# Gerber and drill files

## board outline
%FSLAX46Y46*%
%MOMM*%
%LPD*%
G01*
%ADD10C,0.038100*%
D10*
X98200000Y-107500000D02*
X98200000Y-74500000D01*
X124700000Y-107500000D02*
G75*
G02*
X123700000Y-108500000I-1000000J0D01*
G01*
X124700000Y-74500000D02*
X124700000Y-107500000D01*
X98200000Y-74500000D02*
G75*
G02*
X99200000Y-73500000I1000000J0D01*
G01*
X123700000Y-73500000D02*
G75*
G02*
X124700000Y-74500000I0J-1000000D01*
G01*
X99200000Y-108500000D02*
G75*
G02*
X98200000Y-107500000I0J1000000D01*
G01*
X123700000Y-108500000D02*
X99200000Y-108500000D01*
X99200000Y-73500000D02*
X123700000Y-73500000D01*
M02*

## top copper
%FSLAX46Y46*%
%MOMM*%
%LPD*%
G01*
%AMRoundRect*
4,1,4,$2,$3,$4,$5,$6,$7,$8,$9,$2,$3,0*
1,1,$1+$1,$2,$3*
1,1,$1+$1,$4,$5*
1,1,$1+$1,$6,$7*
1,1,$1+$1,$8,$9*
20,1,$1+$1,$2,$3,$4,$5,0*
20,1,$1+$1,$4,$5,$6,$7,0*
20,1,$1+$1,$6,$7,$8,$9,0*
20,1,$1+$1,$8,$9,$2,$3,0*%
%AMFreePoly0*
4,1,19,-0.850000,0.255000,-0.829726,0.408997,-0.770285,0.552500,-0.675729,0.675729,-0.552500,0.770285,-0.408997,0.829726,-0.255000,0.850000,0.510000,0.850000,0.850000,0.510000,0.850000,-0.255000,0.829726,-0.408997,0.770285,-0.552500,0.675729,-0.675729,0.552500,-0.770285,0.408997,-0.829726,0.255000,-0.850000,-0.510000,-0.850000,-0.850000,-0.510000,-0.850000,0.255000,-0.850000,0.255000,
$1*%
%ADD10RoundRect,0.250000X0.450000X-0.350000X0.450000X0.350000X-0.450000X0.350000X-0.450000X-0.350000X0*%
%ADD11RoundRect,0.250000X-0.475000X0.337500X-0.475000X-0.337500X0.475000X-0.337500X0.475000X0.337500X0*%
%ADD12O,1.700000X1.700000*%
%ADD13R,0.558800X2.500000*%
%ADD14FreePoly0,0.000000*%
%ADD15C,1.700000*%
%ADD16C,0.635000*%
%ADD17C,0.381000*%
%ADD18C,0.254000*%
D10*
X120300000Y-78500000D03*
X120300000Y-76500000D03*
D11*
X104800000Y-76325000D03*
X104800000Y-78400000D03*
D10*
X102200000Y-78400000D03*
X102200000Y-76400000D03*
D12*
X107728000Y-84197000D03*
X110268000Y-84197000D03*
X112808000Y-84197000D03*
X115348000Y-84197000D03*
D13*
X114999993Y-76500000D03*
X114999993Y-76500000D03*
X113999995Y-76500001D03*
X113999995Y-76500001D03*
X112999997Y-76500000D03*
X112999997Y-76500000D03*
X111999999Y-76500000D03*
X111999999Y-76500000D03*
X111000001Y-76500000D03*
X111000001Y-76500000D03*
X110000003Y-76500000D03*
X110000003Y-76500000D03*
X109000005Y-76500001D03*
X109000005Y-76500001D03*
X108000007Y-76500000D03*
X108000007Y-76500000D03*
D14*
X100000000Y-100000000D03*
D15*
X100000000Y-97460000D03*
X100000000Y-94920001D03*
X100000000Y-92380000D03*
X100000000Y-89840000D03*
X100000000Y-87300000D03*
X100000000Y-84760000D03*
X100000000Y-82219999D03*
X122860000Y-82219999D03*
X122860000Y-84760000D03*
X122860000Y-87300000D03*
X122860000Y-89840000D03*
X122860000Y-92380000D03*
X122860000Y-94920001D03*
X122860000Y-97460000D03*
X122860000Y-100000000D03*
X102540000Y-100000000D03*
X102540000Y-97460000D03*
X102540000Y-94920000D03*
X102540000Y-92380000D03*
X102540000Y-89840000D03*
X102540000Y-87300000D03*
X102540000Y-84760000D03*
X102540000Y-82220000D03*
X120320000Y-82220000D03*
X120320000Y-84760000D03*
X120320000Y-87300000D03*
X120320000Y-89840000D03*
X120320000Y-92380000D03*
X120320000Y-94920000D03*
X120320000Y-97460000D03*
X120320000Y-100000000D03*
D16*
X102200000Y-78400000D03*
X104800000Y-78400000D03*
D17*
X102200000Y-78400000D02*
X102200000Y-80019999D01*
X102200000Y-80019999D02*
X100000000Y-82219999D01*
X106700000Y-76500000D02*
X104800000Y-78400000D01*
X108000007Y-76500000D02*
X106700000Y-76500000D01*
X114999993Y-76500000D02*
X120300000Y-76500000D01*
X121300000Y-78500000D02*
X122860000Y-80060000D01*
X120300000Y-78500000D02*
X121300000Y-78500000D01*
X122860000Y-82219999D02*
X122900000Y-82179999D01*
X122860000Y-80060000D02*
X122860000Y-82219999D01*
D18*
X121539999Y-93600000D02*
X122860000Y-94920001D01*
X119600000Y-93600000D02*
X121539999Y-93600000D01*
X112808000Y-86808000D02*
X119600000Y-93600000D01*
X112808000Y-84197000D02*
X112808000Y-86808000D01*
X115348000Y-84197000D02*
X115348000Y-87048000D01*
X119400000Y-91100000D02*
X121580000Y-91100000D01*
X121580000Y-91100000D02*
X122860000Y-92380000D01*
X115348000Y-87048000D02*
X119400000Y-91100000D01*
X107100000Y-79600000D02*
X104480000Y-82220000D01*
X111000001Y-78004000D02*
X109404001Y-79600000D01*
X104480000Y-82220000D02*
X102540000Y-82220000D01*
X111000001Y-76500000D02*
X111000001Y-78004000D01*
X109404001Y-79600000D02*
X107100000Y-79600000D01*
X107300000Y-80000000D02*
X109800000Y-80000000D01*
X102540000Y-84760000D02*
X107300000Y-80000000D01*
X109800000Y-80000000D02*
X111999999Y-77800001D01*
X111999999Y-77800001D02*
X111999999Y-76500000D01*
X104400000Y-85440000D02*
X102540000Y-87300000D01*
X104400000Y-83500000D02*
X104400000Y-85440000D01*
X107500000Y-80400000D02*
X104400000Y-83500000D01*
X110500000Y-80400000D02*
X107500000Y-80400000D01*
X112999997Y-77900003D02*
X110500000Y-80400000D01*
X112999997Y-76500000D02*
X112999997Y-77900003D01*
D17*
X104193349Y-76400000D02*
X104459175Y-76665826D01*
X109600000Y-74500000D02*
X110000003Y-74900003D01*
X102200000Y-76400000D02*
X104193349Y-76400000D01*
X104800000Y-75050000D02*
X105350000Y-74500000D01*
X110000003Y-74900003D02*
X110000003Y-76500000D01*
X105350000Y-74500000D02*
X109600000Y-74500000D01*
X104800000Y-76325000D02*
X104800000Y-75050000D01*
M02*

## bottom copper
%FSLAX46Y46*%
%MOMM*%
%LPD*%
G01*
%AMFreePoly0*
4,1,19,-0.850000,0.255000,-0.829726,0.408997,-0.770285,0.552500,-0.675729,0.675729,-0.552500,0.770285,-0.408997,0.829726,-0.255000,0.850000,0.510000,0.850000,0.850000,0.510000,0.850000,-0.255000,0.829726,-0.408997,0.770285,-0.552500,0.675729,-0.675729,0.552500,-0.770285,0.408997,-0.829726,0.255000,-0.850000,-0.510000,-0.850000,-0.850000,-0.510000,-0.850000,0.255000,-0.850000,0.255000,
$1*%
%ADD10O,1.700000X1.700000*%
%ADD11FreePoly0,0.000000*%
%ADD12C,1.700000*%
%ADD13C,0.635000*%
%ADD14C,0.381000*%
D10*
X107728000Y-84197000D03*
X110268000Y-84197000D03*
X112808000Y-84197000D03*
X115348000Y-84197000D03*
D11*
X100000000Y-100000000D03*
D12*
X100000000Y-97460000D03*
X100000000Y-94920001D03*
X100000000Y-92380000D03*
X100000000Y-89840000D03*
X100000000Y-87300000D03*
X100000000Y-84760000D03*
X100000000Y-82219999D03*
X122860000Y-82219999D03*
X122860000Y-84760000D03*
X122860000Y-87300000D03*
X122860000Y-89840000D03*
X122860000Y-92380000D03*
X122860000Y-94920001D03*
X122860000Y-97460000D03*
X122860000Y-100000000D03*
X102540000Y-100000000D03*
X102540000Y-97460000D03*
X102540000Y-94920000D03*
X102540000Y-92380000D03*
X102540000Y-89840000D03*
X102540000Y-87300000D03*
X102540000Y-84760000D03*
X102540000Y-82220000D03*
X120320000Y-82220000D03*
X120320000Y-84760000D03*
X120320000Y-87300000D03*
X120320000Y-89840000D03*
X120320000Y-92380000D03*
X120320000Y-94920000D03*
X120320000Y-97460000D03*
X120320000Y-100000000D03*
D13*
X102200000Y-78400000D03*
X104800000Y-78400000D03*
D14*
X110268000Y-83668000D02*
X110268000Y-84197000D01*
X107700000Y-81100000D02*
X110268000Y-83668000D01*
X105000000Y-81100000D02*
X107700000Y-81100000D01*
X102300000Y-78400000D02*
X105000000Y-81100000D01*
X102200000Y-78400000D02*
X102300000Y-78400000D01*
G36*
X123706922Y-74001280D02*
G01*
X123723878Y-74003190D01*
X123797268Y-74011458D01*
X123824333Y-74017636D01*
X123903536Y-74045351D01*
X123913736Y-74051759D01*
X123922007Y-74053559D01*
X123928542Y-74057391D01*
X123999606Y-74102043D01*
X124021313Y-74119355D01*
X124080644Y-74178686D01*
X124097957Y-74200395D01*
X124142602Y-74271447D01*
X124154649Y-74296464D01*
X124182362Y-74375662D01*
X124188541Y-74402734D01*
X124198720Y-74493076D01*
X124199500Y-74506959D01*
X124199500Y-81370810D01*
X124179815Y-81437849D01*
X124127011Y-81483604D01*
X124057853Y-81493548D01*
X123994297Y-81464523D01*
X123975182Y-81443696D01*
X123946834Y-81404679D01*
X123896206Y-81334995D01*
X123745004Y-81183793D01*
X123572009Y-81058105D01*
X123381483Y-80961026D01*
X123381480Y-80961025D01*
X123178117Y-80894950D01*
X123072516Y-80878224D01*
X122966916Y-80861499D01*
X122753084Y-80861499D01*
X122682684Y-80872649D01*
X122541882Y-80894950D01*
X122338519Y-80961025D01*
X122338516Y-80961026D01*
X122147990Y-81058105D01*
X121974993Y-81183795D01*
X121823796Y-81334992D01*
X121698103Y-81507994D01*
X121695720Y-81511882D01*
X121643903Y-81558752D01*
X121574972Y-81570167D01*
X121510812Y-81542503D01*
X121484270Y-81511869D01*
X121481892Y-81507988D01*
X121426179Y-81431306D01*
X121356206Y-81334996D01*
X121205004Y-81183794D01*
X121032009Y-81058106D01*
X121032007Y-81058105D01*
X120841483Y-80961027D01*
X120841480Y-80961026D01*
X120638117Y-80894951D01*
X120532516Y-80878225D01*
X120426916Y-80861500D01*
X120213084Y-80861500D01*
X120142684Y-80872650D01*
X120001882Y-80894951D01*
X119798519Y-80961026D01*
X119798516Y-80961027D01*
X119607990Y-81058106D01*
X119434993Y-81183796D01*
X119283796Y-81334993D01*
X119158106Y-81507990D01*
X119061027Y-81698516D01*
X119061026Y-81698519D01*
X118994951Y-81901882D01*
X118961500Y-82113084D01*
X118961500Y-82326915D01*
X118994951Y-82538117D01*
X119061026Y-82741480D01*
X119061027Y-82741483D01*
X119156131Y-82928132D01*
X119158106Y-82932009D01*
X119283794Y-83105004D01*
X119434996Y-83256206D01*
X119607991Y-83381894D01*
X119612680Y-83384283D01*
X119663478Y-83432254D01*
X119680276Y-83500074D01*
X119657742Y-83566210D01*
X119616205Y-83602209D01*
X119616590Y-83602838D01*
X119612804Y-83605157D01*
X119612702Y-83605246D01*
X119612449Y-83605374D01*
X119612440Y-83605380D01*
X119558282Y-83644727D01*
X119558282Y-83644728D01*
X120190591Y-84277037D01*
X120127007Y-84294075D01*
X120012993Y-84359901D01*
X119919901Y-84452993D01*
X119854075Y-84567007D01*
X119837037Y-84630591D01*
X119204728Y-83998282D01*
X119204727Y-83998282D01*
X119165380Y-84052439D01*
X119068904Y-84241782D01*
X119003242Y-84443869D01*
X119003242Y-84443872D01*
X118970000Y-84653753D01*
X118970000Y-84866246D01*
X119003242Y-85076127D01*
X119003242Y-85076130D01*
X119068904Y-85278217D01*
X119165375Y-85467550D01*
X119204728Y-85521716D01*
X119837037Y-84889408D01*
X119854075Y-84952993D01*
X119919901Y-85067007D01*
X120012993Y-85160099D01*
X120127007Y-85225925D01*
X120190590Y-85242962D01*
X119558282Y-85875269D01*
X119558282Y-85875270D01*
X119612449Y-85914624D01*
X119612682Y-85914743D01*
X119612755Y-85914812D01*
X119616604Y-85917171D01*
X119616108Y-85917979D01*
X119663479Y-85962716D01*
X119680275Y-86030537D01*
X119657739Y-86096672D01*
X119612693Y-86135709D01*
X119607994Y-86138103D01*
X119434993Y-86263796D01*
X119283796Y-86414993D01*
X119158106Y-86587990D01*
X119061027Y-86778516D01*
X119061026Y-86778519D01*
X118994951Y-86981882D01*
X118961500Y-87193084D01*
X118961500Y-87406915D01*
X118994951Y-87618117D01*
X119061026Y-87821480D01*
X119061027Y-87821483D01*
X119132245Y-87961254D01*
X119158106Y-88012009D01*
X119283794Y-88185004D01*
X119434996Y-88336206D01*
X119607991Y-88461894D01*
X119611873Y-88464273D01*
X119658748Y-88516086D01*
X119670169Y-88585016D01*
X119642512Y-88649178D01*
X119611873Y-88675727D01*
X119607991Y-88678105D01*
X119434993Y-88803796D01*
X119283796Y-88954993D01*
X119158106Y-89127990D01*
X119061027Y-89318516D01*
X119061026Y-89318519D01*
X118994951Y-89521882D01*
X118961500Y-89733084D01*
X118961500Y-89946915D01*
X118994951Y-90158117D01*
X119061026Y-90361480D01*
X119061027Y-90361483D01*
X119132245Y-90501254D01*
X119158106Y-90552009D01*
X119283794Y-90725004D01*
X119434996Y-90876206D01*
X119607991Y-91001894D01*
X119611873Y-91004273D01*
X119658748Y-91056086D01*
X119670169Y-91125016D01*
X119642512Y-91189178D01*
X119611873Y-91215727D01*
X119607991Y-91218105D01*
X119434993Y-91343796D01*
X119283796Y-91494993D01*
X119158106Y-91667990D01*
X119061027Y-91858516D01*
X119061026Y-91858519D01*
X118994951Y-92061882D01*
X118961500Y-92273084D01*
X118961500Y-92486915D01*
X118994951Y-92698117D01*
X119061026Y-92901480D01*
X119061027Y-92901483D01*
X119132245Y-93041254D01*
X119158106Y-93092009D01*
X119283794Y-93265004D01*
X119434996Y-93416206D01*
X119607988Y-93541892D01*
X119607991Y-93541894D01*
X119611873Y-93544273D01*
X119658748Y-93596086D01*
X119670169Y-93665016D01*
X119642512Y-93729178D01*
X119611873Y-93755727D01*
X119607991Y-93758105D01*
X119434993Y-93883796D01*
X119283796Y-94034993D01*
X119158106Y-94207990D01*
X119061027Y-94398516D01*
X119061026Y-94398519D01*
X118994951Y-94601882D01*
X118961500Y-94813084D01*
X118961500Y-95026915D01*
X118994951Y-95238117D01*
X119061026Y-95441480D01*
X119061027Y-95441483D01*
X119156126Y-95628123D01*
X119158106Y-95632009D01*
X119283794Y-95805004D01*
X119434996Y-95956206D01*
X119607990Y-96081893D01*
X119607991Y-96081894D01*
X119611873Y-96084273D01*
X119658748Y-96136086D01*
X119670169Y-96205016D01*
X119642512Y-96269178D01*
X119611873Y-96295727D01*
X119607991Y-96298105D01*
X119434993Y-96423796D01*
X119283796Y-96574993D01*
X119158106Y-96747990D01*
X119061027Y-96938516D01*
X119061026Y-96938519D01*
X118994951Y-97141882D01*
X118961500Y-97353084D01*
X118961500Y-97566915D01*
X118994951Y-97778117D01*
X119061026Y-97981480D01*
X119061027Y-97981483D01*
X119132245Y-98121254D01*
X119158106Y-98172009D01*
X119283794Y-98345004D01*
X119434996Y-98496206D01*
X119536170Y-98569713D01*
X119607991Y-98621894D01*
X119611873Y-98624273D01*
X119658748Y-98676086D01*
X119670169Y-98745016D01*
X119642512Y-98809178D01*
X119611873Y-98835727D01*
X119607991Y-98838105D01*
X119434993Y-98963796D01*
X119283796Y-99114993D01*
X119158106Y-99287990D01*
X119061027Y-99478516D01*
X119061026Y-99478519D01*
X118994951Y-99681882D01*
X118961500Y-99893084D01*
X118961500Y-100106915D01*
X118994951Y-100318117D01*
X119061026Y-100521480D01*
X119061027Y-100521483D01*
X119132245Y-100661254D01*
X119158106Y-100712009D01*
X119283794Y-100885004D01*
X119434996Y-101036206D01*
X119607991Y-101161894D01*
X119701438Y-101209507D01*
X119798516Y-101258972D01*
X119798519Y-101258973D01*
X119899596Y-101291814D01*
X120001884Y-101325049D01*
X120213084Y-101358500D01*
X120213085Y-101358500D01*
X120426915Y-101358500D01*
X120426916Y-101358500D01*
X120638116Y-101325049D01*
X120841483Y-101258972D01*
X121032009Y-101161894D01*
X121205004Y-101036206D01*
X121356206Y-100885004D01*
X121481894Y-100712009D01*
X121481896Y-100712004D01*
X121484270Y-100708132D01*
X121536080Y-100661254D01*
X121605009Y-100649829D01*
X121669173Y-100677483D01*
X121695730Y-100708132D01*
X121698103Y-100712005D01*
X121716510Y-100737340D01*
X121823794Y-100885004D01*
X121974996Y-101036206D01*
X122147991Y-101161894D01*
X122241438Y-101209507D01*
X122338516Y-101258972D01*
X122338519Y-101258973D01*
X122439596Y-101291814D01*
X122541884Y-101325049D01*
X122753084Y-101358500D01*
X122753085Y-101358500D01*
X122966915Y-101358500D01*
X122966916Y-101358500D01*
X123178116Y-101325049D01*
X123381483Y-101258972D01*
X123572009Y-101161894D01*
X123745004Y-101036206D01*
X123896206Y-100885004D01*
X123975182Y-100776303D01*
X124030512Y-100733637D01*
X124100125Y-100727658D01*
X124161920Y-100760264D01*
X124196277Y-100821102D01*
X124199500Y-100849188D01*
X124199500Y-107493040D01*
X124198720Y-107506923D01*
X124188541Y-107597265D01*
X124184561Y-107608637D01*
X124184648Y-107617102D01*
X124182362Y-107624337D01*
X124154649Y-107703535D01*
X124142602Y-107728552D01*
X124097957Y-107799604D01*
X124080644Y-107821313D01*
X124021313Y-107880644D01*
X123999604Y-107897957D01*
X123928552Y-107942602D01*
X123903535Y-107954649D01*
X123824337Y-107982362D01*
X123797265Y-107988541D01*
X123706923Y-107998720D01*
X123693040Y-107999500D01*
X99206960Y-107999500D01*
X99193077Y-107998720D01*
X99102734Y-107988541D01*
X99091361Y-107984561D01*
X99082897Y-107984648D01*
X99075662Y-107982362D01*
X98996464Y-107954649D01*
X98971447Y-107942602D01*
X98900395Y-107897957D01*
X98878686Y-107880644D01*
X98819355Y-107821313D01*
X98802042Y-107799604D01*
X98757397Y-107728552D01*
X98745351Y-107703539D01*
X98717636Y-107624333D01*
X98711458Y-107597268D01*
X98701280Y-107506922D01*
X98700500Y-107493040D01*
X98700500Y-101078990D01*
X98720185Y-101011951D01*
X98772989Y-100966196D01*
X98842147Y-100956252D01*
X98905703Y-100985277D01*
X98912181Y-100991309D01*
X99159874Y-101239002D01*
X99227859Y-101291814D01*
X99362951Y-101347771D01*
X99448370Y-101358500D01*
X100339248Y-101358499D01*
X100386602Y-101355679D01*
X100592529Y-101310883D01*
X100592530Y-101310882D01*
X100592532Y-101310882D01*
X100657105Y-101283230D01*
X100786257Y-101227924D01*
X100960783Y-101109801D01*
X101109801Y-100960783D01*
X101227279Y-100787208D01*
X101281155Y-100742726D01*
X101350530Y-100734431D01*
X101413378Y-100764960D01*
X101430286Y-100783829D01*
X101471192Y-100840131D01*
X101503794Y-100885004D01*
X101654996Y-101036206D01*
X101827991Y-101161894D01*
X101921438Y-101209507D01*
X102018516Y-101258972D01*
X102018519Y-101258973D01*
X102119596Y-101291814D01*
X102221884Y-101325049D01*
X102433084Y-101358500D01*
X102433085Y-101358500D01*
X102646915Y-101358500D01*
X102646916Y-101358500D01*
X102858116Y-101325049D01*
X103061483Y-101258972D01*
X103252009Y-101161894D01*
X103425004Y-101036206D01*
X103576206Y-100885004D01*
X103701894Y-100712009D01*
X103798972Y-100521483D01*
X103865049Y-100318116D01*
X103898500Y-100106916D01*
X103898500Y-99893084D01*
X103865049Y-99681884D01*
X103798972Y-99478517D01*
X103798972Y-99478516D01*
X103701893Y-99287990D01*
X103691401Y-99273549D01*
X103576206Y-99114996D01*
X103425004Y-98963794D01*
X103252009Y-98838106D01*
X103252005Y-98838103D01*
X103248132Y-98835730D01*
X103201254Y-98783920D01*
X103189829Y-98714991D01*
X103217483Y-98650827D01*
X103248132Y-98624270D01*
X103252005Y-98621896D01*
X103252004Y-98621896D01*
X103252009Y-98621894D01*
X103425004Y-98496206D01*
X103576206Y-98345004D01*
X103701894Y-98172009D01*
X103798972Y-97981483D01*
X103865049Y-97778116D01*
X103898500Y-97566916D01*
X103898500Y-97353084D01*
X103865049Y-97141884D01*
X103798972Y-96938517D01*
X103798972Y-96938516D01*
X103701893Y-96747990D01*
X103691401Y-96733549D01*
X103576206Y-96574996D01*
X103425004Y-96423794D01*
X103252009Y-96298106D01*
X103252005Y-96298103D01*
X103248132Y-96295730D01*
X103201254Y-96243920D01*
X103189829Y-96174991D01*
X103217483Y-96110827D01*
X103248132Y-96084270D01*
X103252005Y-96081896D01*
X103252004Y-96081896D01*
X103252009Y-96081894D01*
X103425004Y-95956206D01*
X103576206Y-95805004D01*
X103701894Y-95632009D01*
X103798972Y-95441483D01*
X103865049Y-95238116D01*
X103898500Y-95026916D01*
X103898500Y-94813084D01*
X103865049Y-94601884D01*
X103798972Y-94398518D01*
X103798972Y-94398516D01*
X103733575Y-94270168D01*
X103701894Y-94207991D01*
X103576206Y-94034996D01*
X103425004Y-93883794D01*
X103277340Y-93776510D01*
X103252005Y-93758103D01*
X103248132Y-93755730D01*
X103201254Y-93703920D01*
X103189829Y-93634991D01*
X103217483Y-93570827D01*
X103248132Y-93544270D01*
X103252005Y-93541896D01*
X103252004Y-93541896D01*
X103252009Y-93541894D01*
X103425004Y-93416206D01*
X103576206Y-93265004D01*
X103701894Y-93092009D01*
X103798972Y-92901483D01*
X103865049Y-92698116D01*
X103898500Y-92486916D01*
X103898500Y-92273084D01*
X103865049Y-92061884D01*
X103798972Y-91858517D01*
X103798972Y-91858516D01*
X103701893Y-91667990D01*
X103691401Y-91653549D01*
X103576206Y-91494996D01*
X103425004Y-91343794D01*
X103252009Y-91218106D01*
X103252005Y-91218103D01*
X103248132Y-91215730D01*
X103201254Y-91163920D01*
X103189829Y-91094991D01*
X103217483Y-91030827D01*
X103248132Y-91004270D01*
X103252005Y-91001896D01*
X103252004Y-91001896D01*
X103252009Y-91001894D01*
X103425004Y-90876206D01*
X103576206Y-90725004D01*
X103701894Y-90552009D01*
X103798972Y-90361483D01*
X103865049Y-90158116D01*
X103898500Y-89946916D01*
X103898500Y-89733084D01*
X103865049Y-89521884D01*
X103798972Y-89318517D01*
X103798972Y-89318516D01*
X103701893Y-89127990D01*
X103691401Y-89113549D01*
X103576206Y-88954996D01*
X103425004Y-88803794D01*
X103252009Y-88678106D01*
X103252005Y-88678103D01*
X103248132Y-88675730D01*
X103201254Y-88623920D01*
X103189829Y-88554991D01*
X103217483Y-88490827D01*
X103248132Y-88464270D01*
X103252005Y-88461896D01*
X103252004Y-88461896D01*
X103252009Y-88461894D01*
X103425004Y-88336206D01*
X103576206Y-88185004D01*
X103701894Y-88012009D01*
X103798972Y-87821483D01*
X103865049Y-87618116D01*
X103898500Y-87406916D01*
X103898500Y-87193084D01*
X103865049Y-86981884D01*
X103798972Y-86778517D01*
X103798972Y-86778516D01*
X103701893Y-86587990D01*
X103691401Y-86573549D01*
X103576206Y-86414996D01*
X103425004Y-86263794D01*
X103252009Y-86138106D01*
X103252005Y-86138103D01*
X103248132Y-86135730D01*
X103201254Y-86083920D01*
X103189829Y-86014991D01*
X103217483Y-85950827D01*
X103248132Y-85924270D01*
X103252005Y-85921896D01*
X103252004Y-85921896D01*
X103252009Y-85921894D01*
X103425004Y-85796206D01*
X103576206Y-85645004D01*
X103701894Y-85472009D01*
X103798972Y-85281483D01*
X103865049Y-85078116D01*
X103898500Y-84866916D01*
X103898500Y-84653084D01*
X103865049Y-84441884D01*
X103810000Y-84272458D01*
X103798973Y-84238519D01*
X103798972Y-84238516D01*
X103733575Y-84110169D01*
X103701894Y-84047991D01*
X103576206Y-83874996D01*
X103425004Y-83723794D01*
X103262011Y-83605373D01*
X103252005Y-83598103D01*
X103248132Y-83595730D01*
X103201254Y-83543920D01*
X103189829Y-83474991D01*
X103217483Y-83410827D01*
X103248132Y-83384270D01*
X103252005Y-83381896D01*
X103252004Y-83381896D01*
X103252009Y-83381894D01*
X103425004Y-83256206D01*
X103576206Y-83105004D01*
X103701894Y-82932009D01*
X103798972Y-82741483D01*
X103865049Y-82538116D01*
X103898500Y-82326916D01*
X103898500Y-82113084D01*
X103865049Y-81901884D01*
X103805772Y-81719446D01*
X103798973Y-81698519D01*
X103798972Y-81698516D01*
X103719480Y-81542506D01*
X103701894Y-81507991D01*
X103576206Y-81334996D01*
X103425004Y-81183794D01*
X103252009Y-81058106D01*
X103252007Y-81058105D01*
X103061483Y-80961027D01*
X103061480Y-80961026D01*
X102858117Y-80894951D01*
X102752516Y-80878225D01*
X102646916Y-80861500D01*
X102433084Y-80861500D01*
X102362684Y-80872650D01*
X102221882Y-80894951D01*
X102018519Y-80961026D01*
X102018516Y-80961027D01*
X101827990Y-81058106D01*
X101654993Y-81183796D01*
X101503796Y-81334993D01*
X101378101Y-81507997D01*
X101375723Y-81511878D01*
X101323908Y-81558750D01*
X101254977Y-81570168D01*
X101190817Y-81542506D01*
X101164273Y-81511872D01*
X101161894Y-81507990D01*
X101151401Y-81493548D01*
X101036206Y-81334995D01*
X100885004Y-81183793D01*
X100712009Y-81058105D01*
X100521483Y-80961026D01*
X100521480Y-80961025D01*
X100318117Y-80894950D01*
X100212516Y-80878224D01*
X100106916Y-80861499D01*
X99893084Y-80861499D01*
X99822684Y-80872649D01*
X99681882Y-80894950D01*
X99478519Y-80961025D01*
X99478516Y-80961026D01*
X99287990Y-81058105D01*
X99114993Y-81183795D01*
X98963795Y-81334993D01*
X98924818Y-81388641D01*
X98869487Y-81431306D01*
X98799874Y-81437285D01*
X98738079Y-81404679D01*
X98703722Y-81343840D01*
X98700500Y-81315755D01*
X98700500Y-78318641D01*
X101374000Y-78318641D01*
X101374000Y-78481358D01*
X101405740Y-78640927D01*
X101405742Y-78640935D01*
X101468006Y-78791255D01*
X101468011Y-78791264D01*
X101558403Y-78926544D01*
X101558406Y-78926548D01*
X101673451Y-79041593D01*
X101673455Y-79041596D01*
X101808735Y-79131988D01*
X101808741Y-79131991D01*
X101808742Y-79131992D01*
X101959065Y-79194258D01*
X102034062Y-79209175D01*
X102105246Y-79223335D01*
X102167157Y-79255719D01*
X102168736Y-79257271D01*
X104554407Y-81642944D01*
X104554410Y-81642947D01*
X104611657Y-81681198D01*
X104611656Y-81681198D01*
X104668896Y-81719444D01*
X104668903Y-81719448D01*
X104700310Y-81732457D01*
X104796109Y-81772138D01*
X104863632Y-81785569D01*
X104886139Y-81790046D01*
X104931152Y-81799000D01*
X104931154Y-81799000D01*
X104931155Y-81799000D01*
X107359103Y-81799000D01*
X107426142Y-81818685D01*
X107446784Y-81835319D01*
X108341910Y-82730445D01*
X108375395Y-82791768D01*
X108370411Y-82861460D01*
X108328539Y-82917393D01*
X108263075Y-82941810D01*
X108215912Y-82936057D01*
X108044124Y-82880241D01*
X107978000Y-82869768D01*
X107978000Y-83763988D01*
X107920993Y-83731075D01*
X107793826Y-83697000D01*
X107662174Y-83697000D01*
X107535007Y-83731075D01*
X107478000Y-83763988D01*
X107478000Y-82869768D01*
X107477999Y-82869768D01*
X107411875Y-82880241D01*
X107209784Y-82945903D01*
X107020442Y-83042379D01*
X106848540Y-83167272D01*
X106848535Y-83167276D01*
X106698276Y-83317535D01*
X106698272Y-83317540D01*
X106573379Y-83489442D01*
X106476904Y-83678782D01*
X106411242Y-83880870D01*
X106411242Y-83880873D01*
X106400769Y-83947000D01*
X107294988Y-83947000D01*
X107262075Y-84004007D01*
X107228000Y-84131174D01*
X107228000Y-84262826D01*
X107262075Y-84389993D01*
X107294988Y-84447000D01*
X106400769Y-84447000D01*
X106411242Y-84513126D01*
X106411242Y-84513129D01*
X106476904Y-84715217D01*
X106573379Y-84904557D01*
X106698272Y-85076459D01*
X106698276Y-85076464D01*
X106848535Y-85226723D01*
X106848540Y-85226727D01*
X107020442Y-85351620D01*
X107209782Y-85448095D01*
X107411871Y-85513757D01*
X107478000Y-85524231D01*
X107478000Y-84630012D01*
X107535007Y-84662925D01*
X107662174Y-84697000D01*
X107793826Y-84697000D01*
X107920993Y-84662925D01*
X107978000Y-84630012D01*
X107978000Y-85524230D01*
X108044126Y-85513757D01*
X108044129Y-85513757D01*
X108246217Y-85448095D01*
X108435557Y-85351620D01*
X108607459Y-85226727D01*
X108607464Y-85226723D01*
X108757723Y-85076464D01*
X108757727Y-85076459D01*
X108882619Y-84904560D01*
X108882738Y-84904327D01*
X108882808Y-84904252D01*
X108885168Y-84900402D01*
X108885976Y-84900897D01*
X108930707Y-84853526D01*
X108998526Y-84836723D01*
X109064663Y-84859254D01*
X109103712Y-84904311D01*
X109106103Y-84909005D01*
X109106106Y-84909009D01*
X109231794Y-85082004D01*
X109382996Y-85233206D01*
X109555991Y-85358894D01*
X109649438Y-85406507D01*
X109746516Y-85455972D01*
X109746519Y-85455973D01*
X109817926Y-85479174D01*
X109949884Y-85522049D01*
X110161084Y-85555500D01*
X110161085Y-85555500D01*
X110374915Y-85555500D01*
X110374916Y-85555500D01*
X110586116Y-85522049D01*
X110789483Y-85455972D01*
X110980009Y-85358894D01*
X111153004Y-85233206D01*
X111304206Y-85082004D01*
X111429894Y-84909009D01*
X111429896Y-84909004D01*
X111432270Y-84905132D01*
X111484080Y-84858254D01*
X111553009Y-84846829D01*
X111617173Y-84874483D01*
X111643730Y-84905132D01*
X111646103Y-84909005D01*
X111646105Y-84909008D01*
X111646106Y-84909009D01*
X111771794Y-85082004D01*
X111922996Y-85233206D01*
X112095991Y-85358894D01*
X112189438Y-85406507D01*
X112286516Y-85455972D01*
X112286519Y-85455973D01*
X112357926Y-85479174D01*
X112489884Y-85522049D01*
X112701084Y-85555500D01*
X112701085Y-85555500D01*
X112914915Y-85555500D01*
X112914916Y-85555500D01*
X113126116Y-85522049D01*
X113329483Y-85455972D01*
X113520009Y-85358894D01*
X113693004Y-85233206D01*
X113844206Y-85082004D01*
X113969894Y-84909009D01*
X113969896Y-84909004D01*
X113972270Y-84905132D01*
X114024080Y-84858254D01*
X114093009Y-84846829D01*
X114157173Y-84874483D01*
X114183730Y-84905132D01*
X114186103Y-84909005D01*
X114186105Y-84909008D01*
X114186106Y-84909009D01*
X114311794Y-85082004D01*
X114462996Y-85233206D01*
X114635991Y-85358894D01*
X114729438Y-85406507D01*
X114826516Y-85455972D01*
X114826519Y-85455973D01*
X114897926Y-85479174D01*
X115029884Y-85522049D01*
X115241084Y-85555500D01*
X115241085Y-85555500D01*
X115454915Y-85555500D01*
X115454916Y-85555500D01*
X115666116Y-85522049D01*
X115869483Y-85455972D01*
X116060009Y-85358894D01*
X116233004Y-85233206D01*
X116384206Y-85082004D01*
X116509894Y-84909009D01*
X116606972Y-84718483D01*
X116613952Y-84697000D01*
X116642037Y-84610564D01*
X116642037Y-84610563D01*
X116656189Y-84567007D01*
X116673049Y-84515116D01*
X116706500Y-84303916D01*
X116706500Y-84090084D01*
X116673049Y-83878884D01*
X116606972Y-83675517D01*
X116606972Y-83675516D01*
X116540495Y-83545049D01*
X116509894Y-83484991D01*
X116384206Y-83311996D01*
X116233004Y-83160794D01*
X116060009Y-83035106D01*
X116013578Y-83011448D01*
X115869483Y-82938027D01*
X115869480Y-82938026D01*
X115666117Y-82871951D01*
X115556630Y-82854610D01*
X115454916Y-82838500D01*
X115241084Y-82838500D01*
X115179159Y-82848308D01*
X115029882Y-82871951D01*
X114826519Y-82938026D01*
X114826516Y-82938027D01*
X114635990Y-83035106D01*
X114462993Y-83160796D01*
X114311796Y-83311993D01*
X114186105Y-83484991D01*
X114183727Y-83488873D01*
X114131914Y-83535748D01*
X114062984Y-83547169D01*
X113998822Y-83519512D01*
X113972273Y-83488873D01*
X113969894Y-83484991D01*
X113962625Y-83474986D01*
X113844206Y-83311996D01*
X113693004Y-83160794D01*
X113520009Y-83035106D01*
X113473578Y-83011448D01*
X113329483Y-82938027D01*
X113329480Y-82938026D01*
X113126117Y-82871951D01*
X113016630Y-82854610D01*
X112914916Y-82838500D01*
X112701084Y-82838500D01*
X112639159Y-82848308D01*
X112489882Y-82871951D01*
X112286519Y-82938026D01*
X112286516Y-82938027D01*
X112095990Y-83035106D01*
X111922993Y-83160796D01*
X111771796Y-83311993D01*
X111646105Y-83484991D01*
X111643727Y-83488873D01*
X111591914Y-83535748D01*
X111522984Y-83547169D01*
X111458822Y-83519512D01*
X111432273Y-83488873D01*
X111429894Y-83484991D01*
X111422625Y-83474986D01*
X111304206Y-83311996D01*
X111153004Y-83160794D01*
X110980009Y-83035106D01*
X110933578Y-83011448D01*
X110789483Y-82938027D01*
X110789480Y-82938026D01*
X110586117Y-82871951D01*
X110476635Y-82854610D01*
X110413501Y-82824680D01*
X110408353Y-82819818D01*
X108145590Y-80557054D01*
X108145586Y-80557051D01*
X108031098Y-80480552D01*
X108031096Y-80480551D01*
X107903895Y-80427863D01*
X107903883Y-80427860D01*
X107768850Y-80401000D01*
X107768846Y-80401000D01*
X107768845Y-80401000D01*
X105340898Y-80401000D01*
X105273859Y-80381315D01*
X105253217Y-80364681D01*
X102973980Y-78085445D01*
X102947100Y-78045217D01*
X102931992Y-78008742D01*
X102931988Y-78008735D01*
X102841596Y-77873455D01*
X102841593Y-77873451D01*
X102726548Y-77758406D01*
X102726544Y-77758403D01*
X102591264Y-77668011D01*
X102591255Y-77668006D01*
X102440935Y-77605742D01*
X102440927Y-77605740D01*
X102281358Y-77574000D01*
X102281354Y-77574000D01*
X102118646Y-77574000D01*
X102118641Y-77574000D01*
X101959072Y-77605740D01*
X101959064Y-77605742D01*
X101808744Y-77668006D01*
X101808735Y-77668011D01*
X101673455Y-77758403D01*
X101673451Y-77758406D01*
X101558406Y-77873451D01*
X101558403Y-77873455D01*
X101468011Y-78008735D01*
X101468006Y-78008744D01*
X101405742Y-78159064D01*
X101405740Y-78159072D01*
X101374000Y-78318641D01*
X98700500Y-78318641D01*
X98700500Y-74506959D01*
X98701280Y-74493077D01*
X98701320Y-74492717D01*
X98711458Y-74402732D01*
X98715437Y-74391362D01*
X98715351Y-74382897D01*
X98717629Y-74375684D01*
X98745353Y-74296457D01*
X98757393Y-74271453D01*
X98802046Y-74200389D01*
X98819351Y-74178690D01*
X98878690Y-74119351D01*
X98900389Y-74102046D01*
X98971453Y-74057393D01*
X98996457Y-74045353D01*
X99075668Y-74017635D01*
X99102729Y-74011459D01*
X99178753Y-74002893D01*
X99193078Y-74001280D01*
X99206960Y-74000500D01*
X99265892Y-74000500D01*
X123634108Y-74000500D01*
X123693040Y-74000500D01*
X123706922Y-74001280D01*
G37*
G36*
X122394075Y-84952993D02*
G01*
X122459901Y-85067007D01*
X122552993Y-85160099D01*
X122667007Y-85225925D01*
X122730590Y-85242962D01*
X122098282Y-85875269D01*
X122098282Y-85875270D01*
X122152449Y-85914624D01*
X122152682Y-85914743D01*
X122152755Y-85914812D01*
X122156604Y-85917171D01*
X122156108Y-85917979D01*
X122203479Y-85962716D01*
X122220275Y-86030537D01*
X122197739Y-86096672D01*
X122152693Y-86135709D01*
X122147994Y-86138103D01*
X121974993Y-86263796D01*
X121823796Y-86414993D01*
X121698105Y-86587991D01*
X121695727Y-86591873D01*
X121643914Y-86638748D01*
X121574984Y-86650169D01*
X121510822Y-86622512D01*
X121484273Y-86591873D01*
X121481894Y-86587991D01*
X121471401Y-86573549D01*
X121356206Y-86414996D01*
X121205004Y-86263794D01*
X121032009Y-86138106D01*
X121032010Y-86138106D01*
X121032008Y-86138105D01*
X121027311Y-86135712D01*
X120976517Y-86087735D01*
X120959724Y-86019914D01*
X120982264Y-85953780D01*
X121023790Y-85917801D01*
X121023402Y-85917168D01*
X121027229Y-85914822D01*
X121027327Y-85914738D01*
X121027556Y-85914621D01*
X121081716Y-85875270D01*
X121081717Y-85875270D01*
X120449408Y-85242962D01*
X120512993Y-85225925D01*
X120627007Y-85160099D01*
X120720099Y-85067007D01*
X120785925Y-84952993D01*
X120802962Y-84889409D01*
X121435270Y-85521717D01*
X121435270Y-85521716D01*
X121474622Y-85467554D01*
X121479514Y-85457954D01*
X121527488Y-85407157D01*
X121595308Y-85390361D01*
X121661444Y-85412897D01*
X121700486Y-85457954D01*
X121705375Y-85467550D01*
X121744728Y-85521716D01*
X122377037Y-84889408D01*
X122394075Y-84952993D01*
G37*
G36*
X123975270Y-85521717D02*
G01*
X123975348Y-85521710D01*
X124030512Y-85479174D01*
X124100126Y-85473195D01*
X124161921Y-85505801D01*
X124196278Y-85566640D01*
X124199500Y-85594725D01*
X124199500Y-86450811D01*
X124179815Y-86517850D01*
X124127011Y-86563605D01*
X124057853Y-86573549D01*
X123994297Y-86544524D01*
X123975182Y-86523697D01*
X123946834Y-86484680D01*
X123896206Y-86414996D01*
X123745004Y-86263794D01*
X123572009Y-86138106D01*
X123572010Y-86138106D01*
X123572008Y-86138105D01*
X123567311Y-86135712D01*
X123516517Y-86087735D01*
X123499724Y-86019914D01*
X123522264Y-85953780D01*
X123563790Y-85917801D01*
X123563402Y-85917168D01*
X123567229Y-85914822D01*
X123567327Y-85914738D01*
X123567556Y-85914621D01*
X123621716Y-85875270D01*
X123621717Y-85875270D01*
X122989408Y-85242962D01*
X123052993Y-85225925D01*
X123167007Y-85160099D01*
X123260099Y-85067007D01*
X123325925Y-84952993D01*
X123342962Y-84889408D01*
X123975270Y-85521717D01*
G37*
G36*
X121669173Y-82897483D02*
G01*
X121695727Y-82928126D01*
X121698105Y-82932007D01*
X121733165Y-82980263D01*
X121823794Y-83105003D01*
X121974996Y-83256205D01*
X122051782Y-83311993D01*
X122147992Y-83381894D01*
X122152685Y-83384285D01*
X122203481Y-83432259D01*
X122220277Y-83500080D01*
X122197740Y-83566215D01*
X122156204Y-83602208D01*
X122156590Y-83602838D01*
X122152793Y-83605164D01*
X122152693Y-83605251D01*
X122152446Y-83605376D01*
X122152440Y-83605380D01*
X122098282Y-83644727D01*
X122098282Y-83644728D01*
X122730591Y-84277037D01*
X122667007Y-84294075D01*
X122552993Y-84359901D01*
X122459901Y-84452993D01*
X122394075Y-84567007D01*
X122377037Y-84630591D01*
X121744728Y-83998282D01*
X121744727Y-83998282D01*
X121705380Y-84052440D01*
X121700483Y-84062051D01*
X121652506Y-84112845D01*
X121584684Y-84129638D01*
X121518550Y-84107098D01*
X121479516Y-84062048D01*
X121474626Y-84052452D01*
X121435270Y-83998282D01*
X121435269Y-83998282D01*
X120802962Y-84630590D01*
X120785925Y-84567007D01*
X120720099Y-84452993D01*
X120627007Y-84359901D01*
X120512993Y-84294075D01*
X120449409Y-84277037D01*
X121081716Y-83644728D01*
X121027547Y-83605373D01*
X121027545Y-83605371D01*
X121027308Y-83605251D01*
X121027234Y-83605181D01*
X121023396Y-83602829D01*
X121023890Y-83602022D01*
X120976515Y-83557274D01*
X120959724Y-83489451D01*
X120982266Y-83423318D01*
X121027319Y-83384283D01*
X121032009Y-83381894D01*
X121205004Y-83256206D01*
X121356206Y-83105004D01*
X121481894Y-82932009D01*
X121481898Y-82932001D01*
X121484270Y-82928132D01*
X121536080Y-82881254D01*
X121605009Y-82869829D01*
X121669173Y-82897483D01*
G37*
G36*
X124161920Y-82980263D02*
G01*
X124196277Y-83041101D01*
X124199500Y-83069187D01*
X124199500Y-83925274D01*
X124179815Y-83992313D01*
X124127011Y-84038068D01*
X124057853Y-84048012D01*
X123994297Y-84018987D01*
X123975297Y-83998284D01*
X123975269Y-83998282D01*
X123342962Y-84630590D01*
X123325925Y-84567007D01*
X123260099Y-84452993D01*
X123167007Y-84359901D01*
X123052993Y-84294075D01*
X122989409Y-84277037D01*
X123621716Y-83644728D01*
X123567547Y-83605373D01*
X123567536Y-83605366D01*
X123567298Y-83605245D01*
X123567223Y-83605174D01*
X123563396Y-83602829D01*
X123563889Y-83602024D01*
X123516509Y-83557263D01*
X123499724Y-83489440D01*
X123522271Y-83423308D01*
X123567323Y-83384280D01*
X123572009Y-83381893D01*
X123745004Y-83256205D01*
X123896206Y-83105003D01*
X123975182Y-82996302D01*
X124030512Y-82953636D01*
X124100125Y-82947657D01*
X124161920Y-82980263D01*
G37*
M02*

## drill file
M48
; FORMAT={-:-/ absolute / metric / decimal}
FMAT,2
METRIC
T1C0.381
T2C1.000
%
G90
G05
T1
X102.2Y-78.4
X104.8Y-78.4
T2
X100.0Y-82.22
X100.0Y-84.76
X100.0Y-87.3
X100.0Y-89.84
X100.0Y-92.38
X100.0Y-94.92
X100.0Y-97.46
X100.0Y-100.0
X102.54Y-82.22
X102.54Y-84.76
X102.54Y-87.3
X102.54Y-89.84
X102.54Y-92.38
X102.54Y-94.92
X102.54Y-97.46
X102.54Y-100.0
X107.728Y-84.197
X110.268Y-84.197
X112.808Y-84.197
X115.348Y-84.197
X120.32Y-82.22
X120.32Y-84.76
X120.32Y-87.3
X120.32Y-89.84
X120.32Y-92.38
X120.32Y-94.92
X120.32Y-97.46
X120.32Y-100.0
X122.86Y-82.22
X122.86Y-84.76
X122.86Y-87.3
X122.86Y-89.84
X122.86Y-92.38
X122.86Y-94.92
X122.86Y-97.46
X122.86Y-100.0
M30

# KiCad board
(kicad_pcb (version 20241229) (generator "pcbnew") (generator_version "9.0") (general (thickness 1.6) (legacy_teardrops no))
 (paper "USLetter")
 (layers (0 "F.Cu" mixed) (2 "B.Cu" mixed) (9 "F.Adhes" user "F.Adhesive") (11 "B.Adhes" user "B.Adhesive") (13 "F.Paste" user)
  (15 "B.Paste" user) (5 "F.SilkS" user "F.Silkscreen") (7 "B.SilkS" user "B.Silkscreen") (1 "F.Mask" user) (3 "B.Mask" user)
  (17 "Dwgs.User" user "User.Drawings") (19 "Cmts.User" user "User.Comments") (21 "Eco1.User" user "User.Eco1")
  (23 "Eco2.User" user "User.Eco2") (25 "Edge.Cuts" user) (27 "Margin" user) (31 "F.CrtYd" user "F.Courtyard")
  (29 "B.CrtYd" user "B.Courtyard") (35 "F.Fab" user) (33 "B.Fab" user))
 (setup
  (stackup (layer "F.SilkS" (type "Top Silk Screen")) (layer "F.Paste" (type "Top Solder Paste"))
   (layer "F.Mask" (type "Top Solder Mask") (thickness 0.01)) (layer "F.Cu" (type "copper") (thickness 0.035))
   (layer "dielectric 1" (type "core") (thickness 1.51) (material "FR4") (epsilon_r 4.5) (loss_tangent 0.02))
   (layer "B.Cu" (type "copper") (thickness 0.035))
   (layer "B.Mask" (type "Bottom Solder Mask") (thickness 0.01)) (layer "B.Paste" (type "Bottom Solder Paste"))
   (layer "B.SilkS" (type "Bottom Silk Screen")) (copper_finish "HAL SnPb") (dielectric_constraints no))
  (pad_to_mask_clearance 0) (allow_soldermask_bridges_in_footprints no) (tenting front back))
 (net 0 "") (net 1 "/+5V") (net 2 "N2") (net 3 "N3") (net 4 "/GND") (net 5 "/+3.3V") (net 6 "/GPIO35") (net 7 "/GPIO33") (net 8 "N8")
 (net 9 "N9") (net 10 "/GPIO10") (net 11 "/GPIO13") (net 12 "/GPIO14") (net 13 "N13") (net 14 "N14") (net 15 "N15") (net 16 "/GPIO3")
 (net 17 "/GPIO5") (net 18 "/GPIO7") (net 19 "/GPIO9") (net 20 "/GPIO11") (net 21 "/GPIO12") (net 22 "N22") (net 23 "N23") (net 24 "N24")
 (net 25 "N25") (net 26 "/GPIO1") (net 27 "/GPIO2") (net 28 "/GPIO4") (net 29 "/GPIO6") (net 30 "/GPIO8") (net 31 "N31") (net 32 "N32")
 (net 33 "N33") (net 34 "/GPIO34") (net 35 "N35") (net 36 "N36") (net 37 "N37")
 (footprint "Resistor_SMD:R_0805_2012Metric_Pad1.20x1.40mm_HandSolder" (layer "F.Cu") (at 120.3 77.5 90)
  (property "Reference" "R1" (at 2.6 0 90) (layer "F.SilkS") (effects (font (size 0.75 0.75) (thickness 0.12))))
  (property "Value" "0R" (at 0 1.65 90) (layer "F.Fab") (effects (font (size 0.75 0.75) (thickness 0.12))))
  (pad "1" smd roundrect (at -1 0 90) (size 1.2 1.4) (layers "F.Cu" "F.Mask" "F.Paste") (roundrect_rratio 0.208333) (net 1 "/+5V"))
  (pad "2" smd roundrect (at 1 0 90) (size 1.2 1.4) (layers "F.Cu" "F.Mask" "F.Paste") (roundrect_rratio 0.208333) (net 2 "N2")))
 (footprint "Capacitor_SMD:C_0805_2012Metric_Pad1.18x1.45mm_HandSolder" (layer "F.Cu") (at 104.8 77.3625 -90)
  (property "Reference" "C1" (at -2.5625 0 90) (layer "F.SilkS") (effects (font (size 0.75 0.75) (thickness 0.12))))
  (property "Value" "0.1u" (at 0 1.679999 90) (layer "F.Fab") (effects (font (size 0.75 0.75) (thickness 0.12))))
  (pad "1" smd roundrect (at -1.0375 0 270) (size 1.175 1.45) (layers "F.Cu" "F.Mask" "F.Paste") (roundrect_rratio 0.212766) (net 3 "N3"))
  (pad "2" smd roundrect (at 1.0375 0 270) (size 1.175 1.45) (layers "F.Cu" "F.Mask" "F.Paste") (roundrect_rratio 0.212766) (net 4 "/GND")))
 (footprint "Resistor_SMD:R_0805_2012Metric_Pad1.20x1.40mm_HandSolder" (layer "F.Cu") (at 102.2 77.4 90)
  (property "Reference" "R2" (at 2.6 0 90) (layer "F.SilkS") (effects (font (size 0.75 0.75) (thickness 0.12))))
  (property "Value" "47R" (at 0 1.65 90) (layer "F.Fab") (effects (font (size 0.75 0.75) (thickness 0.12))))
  (pad "1" smd roundrect (at -1 0 90) (size 1.2 1.4) (layers "F.Cu" "F.Mask" "F.Paste") (roundrect_rratio 0.208333) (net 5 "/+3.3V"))
  (pad "2" smd roundrect (at 1 0 90) (size 1.2 1.4) (layers "F.Cu" "F.Mask" "F.Paste") (roundrect_rratio 0.208333) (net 3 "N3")))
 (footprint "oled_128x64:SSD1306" (layer "F.Cu") (at 111.538 93.849)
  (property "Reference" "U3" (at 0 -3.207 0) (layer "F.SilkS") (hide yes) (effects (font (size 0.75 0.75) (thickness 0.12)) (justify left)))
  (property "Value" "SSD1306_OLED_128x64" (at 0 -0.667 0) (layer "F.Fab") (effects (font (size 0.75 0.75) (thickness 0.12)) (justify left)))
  (pad "1" thru_hole oval (at -3.81 -9.652 90) (size 1.7 1.7) (drill oval 1) (layers "*.Cu" "*.Mask") (remove_unused_layers no)
   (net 4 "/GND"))
  (pad "2" thru_hole oval (at -1.27 -9.652 90) (size 1.7 1.7) (drill oval 1) (layers "*.Cu" "*.Mask") (remove_unused_layers no)
   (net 5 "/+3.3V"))
  (pad "3" thru_hole oval (at 1.27 -9.652 90) (size 1.7 1.7) (drill oval 1) (layers "*.Cu" "*.Mask") (remove_unused_layers no)
   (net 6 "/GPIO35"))
  (pad "4" thru_hole oval (at 3.81 -9.652 90) (size 1.7 1.7) (drill oval 1) (layers "*.Cu" "*.Mask") (remove_unused_layers no)
   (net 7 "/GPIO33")))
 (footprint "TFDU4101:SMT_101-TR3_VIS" (layer "F.Cu") (at 111.5 75.6999 90)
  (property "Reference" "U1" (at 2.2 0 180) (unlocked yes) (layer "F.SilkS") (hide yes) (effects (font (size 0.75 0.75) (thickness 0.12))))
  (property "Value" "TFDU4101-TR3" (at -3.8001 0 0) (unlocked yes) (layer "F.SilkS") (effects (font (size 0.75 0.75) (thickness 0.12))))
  (pad "1" smd rect (at -0.8001 3.499993 90) (size 2.5 0.5588) (layers "F.Cu" "F.Mask" "F.Paste") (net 2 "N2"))
  (pad "1" smd rect (at -0.8001 3.499993 90) (size 2.5 0.5588) (layers "F.Cu" "F.Mask" "F.Paste") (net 2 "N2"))
  (pad "2" smd rect (at -0.800101 2.499995 90) (size 2.5 0.5588) (layers "F.Cu" "F.Mask" "F.Paste") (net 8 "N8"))
  (pad "2" smd rect (at -0.800101 2.499995 90) (size 2.5 0.5588) (layers "F.Cu" "F.Mask" "F.Paste") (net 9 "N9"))
  (pad "3" smd rect (at -0.8001 1.499997 90) (size 2.5 0.5588) (layers "F.Cu" "F.Mask" "F.Paste") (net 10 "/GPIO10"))
  (pad "3" smd rect (at -0.8001 1.499997 90) (size 2.5 0.5588) (layers "F.Cu" "F.Mask" "F.Paste") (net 10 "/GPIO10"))
  (pad "4" smd rect (at -0.8001 0.499999 90) (size 2.5 0.5588) (layers "F.Cu" "F.Mask" "F.Paste") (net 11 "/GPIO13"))
  (pad "4" smd rect (at -0.8001 0.499999 90) (size 2.5 0.5588) (layers "F.Cu" "F.Mask" "F.Paste") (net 11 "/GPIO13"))
  (pad "5" smd rect (at -0.8001 -0.499999 90) (size 2.5 0.5588) (layers "F.Cu" "F.Mask" "F.Paste") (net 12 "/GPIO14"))
  (pad "5" smd rect (at -0.8001 -0.499999 90) (size 2.5 0.5588) (layers "F.Cu" "F.Mask" "F.Paste") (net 12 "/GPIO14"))
  (pad "6" smd rect (at -0.8001 -1.499997 90) (size 2.5 0.5588) (layers "F.Cu" "F.Mask" "F.Paste") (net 3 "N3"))
  (pad "6" smd rect (at -0.8001 -1.499997 90) (size 2.5 0.5588) (layers "F.Cu" "F.Mask" "F.Paste") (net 3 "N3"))
  (pad "7" smd rect (at -0.800101 -2.499995 90) (size 2.5 0.5588) (layers "F.Cu" "F.Mask" "F.Paste") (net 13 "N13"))
  (pad "7" smd rect (at -0.800101 -2.499995 90) (size 2.5 0.5588) (layers "F.Cu" "F.Mask" "F.Paste") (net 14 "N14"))
  (pad "8" smd rect (at -0.8001 -3.499993 90) (size 2.5 0.5588) (layers "F.Cu" "F.Mask" "F.Paste") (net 4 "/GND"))
  (pad "8" smd rect (at -0.8001 -3.499993 90) (size 2.5 0.5588) (layers "F.Cu" "F.Mask" "F.Paste") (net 4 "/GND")))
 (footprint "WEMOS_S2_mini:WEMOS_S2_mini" (layer "B.Cu") (at 100 100)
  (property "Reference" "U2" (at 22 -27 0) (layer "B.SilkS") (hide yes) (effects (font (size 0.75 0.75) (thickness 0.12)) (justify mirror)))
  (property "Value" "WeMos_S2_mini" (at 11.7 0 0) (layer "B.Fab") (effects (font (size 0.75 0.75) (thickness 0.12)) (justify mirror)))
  (pad "1" thru_hole roundrect (at 0 0) (size 1.7 1.7) (drill 1) (layers "*.Cu" "*.Mask") (remove_unused_layers no) (roundrect_rratio 0.35)
   (chamfer_ratio 0.2) (chamfer top_right bottom_left) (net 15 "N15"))
  (pad "2" thru_hole circle (at 0 -2.54) (size 1.7 1.7) (drill 1) (layers "*.Cu" "*.Mask") (remove_unused_layers no) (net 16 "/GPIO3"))
  (pad "3" thru_hole circle (at 0 -5.079999) (size 1.7 1.7) (drill 1) (layers "*.Cu" "*.Mask") (remove_unused_layers no) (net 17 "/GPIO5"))
  (pad "4" thru_hole circle (at 0 -7.62) (size 1.7 1.7) (drill 1) (layers "*.Cu" "*.Mask") (remove_unused_layers no) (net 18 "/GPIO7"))
  (pad "5" thru_hole circle (at 0 -10.16) (size 1.7 1.7) (drill 1) (layers "*.Cu" "*.Mask") (remove_unused_layers no) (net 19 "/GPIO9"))
  (pad "6" thru_hole circle (at 0 -12.7) (size 1.7 1.7) (drill 1) (layers "*.Cu" "*.Mask") (remove_unused_layers no) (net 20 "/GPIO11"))
  (pad "7" thru_hole circle (at 0 -15.24) (size 1.7 1.7) (drill 1) (layers "*.Cu" "*.Mask") (remove_unused_layers no) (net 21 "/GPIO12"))
  (pad "8" thru_hole circle (at 0 -17.780001) (size 1.7 1.7) (drill 1) (layers "*.Cu" "*.Mask") (remove_unused_layers no) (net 5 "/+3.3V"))
  (pad "9" thru_hole circle (at 22.86 -17.780001) (size 1.7 1.7) (drill 1) (layers "*.Cu" "*.Mask") (remove_unused_layers no) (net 1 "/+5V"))
  (pad "10" thru_hole circle (at 22.86 -15.24) (size 1.7 1.7) (drill 1) (layers "*.Cu" "*.Mask") (remove_unused_layers no) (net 4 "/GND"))
  (pad "11" thru_hole circle (at 22.86 -12.7) (size 1.7 1.7) (drill 1) (layers "*.Cu" "*.Mask") (remove_unused_layers no) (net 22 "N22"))
  (pad "12" thru_hole circle (at 22.86 -10.16) (size 1.7 1.7) (drill 1) (layers "*.Cu" "*.Mask") (remove_unused_layers no) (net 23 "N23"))
  (pad "13" thru_hole circle (at 22.86 -7.62) (size 1.7 1.7) (drill 1) (layers "*.Cu" "*.Mask") (remove_unused_layers no) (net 7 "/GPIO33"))
  (pad "14" thru_hole circle (at 22.86 -5.079999) (size 1.7 1.7) (drill 1) (layers "*.Cu" "*.Mask") (remove_unused_layers no)
   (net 6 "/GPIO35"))
  (pad "15" thru_hole circle (at 22.86 -2.54) (size 1.7 1.7) (drill 1) (layers "*.Cu" "*.Mask") (remove_unused_layers no) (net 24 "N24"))
  (pad "16" thru_hole circle (at 22.86 0) (size 1.7 1.7) (drill 1) (layers "*.Cu" "*.Mask") (remove_unused_layers no) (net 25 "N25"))
  (pad "17" thru_hole circle (at 2.54 0) (size 1.7 1.7) (drill 1) (layers "*.Cu" "*.Mask") (remove_unused_layers no) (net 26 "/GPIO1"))
  (pad "18" thru_hole circle (at 2.54 -2.54) (size 1.7 1.7) (drill 1) (layers "*.Cu" "*.Mask") (remove_unused_layers no) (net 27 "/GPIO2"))
  (pad "19" thru_hole circle (at 2.54 -5.08) (size 1.7 1.7) (drill 1) (layers "*.Cu" "*.Mask") (remove_unused_layers no) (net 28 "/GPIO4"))
  (pad "20" thru_hole circle (at 2.54 -7.62) (size 1.7 1.7) (drill 1) (layers "*.Cu" "*.Mask") (remove_unused_layers no) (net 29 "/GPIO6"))
  (pad "21" thru_hole circle (at 2.54 -10.16) (size 1.7 1.7) (drill 1) (layers "*.Cu" "*.Mask") (remove_unused_layers no) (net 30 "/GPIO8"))
  (pad "22" thru_hole circle (at 2.54 -12.7) (size 1.7 1.7) (drill 1) (layers "*.Cu" "*.Mask") (remove_unused_layers no) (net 10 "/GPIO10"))
  (pad "23" thru_hole circle (at 2.54 -15.24) (size 1.7 1.7) (drill 1) (layers "*.Cu" "*.Mask") (remove_unused_layers no) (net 11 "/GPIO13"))
  (pad "24" thru_hole circle (at 2.54 -17.78) (size 1.7 1.7) (drill 1) (layers "*.Cu" "*.Mask") (remove_unused_layers no) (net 12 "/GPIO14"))
  (pad "25" thru_hole circle (at 20.32 -17.78) (size 1.7 1.7) (drill 1) (layers "*.Cu" "*.Mask") (remove_unused_layers no) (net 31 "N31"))
  (pad "26" thru_hole circle (at 20.32 -15.24) (size 1.7 1.7) (drill 1) (layers "*.Cu" "*.Mask") (remove_unused_layers no) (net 4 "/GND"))
  (pad "27" thru_hole circle (at 20.32 -12.7) (size 1.7 1.7) (drill 1) (layers "*.Cu" "*.Mask") (remove_unused_layers no) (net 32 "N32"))
  (pad "28" thru_hole circle (at 20.32 -10.16) (size 1.7 1.7) (drill 1) (layers "*.Cu" "*.Mask") (remove_unused_layers no) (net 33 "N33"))
  (pad "29" thru_hole circle (at 20.32 -7.62) (size 1.7 1.7) (drill 1) (layers "*.Cu" "*.Mask") (remove_unused_layers no) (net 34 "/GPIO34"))
  (pad "30" thru_hole circle (at 20.32 -5.08) (size 1.7 1.7) (drill 1) (layers "*.Cu" "*.Mask") (remove_unused_layers no) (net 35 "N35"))
  (pad "31" thru_hole circle (at 20.32 -2.54) (size 1.7 1.7) (drill 1) (layers "*.Cu" "*.Mask") (remove_unused_layers no) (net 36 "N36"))
  (pad "32" thru_hole circle (at 20.32 0) (size 1.7 1.7) (drill 1) (layers "*.Cu" "*.Mask") (remove_unused_layers no) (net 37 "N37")))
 (gr_line (start 98.2 107.5) (end 98.2 74.5) (stroke (width 0.0381) (type default)) (layer "Edge.Cuts"))
 (gr_arc (start 124.7 107.5) (mid 124.407107 108.207107) (end 123.7 108.5) (stroke (width 0.0381) (type default)) (layer "Edge.Cuts"))
 (gr_line (start 124.7 74.5) (end 124.7 107.5) (stroke (width 0.0381) (type default)) (layer "Edge.Cuts"))
 (gr_arc (start 98.2 74.5) (mid 98.492893 73.792893) (end 99.2 73.5) (stroke (width 0.0381) (type default)) (layer "Edge.Cuts"))
 (gr_arc (start 123.7 73.5) (mid 124.407107 73.792893) (end 124.7 74.5) (stroke (width 0.0381) (type default)) (layer "Edge.Cuts"))
 (gr_arc (start 99.2 108.5) (mid 98.492893 108.207107) (end 98.2 107.5) (stroke (width 0.0381) (type default)) (layer "Edge.Cuts"))
 (gr_line (start 123.7 108.5) (end 99.2 108.5) (stroke (width 0.0381) (type default)) (layer "Edge.Cuts"))
 (gr_line (start 99.2 73.5) (end 123.7 73.5) (stroke (width 0.0381) (type default)) (layer "Edge.Cuts"))
 (segment (start 102.2 78.4) (end 102.2 80.019999) (width 0.381) (layer "F.Cu") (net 5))
 (segment (start 102.2 80.019999) (end 100 82.219999) (width 0.381) (layer "F.Cu") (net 5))
 (via (at 102.2 78.4) (size 0.635) (drill 0.381) (layers "F.Cu" "B.Cu") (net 5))
 (segment (start 110.268 83.668) (end 110.268 84.197) (width 0.381) (layer "B.Cu") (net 5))
 (segment (start 107.7 81.1) (end 110.268 83.668) (width 0.381) (layer "B.Cu") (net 5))
 (segment (start 105 81.1) (end 107.7 81.1) (width 0.381) (layer "B.Cu") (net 5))
 (segment (start 102.3 78.4) (end 105 81.1) (width 0.381) (layer "B.Cu") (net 5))
 (segment (start 102.2 78.4) (end 102.3 78.4) (width 0.381) (layer "B.Cu") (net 5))
 (segment (start 106.7 76.5) (end 104.8 78.4) (width 0.381) (layer "F.Cu") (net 4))
 (segment (start 108.000007 76.5) (end 106.7 76.5) (width 0.381) (layer "F.Cu") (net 4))
 (via (at 104.8 78.4) (size 0.635) (drill 0.381) (layers "F.Cu" "B.Cu") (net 4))
 (segment (start 114.999993 76.5) (end 120.3 76.5) (width 0.381) (layer "F.Cu") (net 2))
 (segment (start 121.3 78.5) (end 122.86 80.06) (width 0.381) (layer "F.Cu") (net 1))
 (segment (start 120.3 78.5) (end 121.3 78.5) (width 0.381) (layer "F.Cu") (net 1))
 (segment (start 122.86 82.219999) (end 122.9 82.179999) (width 0.381) (layer "F.Cu") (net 1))
 (segment (start 122.86 80.06) (end 122.86 82.219999) (width 0.381) (layer "F.Cu") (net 1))
 (segment (start 121.539999 93.6) (end 122.86 94.920001) (width 0.254) (layer "F.Cu") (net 6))
 (segment (start 119.6 93.6) (end 121.539999 93.6) (width 0.254) (layer "F.Cu") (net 6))
 (segment (start 112.808 86.808) (end 119.6 93.6) (width 0.254) (layer "F.Cu") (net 6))
 (segment (start 112.808 84.197) (end 112.808 86.808) (width 0.254) (layer "F.Cu") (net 6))
 (segment (start 115.348 84.197) (end 115.348 87.048) (width 0.254) (layer "F.Cu") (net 7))
 (segment (start 119.4 91.1) (end 121.58 91.1) (width 0.254) (layer "F.Cu") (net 7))
 (segment (start 121.58 91.1) (end 122.86 92.38) (width 0.254) (layer "F.Cu") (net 7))
 (segment (start 115.348 87.048) (end 119.4 91.1) (width 0.254) (layer "F.Cu") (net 7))
 (segment (start 107.1 79.6) (end 104.48 82.22) (width 0.254) (layer "F.Cu") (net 12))
 (segment (start 111.000001 78.004) (end 109.404001 79.6) (width 0.254) (layer "F.Cu") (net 12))
 (segment (start 104.48 82.22) (end 102.54 82.22) (width 0.254) (layer "F.Cu") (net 12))
 (segment (start 111.000001 76.5) (end 111.000001 78.004) (width 0.254) (layer "F.Cu") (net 12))
 (segment (start 109.404001 79.6) (end 107.1 79.6) (width 0.254) (layer "F.Cu") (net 12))
 (segment (start 107.3 80) (end 109.8 80) (width 0.254) (layer "F.Cu") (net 11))
 (segment (start 102.54 84.76) (end 107.3 80) (width 0.254) (layer "F.Cu") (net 11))
 (segment (start 109.8 80) (end 111.999999 77.800001) (width 0.254) (layer "F.Cu") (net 11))
 (segment (start 111.999999 77.800001) (end 111.999999 76.5) (width 0.254) (layer "F.Cu") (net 11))
 (segment (start 104.4 85.44) (end 102.54 87.3) (width 0.254) (layer "F.Cu") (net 10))
 (segment (start 104.4 83.5) (end 104.4 85.44) (width 0.254) (layer "F.Cu") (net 10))
 (segment (start 107.5 80.4) (end 104.4 83.5) (width 0.254) (layer "F.Cu") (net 10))
 (segment (start 110.5 80.4) (end 107.5 80.4) (width 0.254) (layer "F.Cu") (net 10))
 (segment (start 112.999997 77.900003) (end 110.5 80.4) (width 0.254) (layer "F.Cu") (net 10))
 (segment (start 112.999997 76.5) (end 112.999997 77.900003) (width 0.254) (layer "F.Cu") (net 10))
 (segment (start 104.193349 76.4) (end 104.459175 76.665826) (width 0.381) (layer "F.Cu") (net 3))
 (segment (start 109.6 74.5) (end 110.000003 74.900003) (width 0.381) (layer "F.Cu") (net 3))
 (segment (start 102.2 76.4) (end 104.193349 76.4) (width 0.381) (layer "F.Cu") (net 3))
 (segment (start 104.8 75.05) (end 105.35 74.5) (width 0.381) (layer "F.Cu") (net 3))
 (segment (start 110.000003 74.900003) (end 110.000003 76.5) (width 0.381) (layer "F.Cu") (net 3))
 (segment (start 105.35 74.5) (end 109.6 74.5) (width 0.381) (layer "F.Cu") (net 3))
 (segment (start 104.8 76.325) (end 104.8 75.05) (width 0.381) (layer "F.Cu") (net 3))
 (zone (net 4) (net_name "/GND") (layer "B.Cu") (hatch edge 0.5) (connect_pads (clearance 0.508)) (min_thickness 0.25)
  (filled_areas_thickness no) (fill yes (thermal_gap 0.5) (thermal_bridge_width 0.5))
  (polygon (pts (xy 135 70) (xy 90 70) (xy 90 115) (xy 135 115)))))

